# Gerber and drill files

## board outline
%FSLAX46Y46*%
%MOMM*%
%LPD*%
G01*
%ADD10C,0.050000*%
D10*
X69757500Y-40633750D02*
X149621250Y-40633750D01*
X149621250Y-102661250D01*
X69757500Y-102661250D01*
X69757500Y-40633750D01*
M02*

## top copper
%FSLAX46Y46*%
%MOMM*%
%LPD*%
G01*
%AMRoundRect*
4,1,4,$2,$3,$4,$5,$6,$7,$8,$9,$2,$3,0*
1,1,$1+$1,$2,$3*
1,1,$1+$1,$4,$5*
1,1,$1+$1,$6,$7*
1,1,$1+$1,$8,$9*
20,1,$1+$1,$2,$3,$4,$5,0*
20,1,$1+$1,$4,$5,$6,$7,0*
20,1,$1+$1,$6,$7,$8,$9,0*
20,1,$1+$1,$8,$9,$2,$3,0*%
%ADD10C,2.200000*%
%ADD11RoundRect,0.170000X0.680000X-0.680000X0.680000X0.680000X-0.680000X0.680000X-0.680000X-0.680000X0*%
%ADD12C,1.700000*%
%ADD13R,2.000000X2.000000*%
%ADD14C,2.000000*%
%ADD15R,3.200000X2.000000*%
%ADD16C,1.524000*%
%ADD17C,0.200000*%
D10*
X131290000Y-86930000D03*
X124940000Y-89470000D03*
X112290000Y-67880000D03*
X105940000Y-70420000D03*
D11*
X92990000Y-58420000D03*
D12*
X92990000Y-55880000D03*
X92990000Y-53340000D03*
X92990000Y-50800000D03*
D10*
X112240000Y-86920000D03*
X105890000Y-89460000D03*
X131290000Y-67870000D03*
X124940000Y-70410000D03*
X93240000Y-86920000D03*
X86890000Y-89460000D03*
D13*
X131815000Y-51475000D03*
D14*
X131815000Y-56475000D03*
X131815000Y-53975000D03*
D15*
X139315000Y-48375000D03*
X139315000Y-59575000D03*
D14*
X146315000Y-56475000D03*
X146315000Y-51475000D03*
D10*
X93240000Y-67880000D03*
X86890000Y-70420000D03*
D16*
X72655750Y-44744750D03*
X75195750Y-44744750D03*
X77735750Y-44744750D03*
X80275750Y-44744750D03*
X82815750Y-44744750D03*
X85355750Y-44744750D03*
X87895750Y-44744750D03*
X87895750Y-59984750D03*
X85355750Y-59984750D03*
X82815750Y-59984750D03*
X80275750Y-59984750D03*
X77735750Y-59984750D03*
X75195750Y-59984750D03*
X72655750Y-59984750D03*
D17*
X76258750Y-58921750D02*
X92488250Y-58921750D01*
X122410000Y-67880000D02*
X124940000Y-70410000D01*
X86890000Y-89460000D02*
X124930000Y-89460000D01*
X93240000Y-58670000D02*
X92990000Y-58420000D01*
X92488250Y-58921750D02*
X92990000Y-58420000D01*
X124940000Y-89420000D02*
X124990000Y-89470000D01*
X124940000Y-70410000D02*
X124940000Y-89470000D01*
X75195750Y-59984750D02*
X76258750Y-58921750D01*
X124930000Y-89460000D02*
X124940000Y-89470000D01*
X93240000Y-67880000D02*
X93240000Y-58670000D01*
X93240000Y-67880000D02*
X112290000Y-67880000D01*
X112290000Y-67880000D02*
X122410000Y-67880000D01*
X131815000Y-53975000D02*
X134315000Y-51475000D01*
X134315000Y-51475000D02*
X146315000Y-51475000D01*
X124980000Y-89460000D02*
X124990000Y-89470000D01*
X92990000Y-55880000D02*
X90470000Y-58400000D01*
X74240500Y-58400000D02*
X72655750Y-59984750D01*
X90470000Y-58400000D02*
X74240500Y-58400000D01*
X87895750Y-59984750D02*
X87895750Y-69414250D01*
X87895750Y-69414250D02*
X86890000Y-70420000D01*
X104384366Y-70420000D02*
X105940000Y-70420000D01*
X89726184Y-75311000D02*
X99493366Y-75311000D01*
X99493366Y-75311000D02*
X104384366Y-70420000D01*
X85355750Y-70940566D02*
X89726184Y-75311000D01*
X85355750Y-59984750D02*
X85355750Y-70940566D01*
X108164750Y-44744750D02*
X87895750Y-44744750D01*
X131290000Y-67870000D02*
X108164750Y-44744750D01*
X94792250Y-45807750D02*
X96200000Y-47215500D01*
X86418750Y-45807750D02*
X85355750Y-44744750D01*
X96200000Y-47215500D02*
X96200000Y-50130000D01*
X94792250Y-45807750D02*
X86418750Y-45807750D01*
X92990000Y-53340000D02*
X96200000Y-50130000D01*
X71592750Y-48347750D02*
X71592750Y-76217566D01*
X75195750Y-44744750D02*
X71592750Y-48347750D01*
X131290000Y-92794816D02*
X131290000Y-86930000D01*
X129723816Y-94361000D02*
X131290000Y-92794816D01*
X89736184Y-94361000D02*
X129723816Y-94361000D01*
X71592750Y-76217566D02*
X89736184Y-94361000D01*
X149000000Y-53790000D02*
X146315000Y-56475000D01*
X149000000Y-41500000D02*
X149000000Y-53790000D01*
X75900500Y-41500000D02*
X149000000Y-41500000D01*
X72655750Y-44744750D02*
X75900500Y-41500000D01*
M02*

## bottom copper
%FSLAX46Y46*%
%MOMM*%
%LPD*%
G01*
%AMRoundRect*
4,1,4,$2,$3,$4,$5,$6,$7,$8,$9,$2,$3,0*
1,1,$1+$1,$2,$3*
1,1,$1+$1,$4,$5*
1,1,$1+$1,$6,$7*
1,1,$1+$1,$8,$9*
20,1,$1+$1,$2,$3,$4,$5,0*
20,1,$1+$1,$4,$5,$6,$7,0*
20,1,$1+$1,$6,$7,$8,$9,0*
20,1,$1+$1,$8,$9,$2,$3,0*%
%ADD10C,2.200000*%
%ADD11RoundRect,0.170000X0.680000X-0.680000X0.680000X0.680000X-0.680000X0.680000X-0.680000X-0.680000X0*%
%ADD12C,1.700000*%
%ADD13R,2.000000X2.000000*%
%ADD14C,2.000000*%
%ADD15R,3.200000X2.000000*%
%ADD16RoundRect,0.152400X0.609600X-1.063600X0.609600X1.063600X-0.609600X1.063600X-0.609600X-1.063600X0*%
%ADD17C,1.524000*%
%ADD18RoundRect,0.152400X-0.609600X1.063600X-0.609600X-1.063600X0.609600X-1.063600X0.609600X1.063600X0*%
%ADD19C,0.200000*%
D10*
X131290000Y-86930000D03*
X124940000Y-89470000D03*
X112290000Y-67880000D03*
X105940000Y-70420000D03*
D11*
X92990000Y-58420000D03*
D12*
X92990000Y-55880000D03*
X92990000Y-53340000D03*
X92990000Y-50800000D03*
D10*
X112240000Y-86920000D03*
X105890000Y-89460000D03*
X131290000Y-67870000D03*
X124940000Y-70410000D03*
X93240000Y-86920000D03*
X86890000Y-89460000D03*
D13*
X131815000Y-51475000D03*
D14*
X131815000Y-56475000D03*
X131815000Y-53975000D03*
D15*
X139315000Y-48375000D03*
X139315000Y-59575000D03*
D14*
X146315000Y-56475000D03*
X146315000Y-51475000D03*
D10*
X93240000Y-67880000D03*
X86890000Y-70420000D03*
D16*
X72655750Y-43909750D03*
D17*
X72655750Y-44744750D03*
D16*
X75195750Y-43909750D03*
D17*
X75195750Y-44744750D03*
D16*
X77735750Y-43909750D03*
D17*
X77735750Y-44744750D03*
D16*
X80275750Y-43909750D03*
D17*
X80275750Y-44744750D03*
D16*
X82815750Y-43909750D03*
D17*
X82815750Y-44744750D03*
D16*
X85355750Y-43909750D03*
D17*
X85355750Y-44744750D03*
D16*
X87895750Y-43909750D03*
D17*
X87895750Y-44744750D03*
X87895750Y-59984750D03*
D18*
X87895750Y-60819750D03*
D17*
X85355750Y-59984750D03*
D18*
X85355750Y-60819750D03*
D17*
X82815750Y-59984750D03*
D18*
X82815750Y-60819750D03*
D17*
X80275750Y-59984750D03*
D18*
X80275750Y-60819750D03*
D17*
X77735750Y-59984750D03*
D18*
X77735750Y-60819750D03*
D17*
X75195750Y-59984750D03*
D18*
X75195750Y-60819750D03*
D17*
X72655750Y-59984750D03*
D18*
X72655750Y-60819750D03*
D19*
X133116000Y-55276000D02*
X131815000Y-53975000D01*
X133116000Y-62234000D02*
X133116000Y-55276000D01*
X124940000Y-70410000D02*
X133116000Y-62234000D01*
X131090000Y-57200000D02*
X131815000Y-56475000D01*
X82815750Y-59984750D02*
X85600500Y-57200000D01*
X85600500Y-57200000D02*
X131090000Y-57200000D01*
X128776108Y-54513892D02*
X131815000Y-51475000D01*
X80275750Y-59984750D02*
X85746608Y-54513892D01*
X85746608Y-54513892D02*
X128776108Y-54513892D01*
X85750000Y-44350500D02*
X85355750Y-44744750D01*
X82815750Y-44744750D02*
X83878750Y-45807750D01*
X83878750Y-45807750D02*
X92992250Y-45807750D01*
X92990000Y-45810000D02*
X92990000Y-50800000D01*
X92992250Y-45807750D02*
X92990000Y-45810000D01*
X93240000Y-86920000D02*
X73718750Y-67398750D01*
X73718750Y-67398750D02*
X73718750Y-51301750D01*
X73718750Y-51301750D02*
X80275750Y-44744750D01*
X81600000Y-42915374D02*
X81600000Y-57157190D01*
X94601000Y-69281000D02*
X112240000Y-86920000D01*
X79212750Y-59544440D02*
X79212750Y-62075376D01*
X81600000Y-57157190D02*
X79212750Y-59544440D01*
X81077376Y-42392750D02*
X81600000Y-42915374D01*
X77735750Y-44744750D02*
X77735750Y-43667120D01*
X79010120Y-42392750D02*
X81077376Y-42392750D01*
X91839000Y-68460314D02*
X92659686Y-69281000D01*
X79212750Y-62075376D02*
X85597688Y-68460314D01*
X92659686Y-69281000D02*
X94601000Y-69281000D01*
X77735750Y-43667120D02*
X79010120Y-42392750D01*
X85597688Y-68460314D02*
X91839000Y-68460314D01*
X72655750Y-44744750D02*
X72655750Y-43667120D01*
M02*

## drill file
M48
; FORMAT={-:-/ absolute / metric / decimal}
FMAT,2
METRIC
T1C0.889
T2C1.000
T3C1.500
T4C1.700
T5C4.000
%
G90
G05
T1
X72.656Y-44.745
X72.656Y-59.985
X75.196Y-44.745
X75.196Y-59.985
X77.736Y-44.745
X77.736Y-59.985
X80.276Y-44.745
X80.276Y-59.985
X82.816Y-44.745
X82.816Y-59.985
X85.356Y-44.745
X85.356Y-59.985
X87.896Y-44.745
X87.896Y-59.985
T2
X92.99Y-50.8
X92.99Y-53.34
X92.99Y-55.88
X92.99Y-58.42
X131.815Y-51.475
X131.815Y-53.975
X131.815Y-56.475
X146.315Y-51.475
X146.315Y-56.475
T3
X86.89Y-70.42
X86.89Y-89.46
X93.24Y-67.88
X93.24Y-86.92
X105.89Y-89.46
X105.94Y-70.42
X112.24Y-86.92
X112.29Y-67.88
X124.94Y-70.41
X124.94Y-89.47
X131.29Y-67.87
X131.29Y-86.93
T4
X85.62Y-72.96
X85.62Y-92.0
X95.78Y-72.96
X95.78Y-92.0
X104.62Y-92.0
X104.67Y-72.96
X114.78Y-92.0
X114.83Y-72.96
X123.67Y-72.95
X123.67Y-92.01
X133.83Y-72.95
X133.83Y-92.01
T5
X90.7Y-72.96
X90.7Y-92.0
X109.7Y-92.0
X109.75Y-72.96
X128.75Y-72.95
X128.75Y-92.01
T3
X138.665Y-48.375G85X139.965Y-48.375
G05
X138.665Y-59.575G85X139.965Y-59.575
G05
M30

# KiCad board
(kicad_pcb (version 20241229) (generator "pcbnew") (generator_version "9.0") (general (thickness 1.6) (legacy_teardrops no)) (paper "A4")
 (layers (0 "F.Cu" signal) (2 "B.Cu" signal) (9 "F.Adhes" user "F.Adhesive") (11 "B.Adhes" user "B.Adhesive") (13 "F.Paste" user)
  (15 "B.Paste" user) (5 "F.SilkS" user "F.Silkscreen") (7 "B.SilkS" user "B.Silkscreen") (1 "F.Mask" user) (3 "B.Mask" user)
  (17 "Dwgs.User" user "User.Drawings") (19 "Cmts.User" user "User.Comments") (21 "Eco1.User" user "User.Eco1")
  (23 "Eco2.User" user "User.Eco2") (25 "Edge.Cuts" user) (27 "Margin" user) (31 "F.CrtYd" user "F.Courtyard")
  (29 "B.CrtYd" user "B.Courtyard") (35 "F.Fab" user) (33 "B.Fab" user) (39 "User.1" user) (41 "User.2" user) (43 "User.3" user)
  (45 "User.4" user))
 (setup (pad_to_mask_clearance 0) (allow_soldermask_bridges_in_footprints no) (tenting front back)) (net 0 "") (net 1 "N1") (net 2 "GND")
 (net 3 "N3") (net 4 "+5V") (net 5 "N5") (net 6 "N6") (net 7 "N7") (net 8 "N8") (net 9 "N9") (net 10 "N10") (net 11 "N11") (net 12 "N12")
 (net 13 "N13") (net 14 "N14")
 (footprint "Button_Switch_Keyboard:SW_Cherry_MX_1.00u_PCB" (layer "F.Cu") (at 131.29 86.93)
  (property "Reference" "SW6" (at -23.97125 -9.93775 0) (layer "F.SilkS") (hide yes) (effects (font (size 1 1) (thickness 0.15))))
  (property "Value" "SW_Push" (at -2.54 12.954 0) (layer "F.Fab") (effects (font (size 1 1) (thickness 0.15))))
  (pad "" np_thru_hole circle (at -7.62 5.08) (size 1.7 1.7) (drill 1.7) (layers "*.Cu" "*.Mask"))
  (pad "" np_thru_hole circle (at -2.54 5.08) (size 4 4) (drill 4) (layers "*.Cu" "*.Mask"))
  (pad "" np_thru_hole circle (at 2.54 5.08) (size 1.7 1.7) (drill 1.7) (layers "*.Cu" "*.Mask"))
  (pad "1" thru_hole circle (at 0 0) (size 2.2 2.2) (drill 1.5) (layers "*.Cu" "*.Mask") (remove_unused_layers no) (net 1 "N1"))
  (pad "2" thru_hole circle (at -6.35 2.54) (size 2.2 2.2) (drill 1.5) (layers "*.Cu" "*.Mask") (remove_unused_layers no) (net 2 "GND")))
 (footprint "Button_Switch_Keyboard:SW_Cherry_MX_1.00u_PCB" (layer "F.Cu") (at 112.29 67.88)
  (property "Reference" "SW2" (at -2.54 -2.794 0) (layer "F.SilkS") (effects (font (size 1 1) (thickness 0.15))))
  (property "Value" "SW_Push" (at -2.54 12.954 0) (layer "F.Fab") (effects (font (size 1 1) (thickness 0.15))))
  (pad "" np_thru_hole circle (at -7.62 5.08) (size 1.7 1.7) (drill 1.7) (layers "*.Cu" "*.Mask"))
  (pad "" np_thru_hole circle (at -2.54 5.08) (size 4 4) (drill 4) (layers "*.Cu" "*.Mask"))
  (pad "" np_thru_hole circle (at 2.54 5.08) (size 1.7 1.7) (drill 1.7) (layers "*.Cu" "*.Mask"))
  (pad "1" thru_hole circle (at 0 0) (size 2.2 2.2) (drill 1.5) (layers "*.Cu" "*.Mask") (remove_unused_layers no) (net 2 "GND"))
  (pad "2" thru_hole circle (at -6.35 2.54) (size 2.2 2.2) (drill 1.5) (layers "*.Cu" "*.Mask") (remove_unused_layers no) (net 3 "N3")))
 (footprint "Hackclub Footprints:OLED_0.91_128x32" (layer "F.Cu") (at 92.99 58.42 90)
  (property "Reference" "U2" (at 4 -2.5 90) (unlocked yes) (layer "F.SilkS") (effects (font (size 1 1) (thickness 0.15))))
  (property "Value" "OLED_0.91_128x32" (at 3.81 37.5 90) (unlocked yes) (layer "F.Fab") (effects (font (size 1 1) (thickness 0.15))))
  (pad "1" thru_hole roundrect (at 0 0 90) (size 1.7 1.7) (drill 1) (layers "*.Cu" "*.Mask") (remove_unused_layers no)
   (roundrect_rratio 0.1) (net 2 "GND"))
  (pad "2" thru_hole circle (at 2.54 0 90) (size 1.7 1.7) (drill 1) (layers "*.Cu" "*.Mask") (remove_unused_layers no) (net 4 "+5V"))
  (pad "3" thru_hole circle (at 5.08 0 90) (size 1.7 1.7) (drill 1) (layers "*.Cu" "*.Mask") (remove_unused_layers no) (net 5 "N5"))
  (pad "4" thru_hole circle (at 7.62 0 90) (size 1.7 1.7) (drill 1) (layers "*.Cu" "*.Mask") (remove_unused_layers no) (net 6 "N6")))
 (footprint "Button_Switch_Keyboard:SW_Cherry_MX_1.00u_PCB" (layer "F.Cu") (at 112.24 86.92)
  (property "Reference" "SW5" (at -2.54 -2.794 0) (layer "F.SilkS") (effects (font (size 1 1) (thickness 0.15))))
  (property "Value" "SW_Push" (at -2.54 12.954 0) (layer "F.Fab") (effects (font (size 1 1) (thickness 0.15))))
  (pad "" np_thru_hole circle (at -7.62 5.08) (size 1.7 1.7) (drill 1.7) (layers "*.Cu" "*.Mask"))
  (pad "" np_thru_hole circle (at -2.54 5.08) (size 4 4) (drill 4) (layers "*.Cu" "*.Mask"))
  (pad "" np_thru_hole circle (at 2.54 5.08) (size 1.7 1.7) (drill 1.7) (layers "*.Cu" "*.Mask"))
  (pad "1" thru_hole circle (at 0 0) (size 2.2 2.2) (drill 1.5) (layers "*.Cu" "*.Mask") (remove_unused_layers no) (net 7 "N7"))
  (pad "2" thru_hole circle (at -6.35 2.54) (size 2.2 2.2) (drill 1.5) (layers "*.Cu" "*.Mask") (remove_unused_layers no) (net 2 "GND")))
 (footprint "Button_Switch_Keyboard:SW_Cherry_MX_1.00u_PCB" (layer "F.Cu") (at 131.29 67.87)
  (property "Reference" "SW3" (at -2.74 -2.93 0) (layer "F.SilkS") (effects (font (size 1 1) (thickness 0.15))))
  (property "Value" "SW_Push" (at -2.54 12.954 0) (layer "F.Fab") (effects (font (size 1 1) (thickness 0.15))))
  (pad "" np_thru_hole circle (at -7.62 5.08) (size 1.7 1.7) (drill 1.7) (layers "*.Cu" "*.Mask"))
  (pad "" np_thru_hole circle (at -2.54 5.08) (size 4 4) (drill 4) (layers "*.Cu" "*.Mask"))
  (pad "" np_thru_hole circle (at 2.54 5.08) (size 1.7 1.7) (drill 1.7) (layers "*.Cu" "*.Mask"))
  (pad "1" thru_hole circle (at 0 0) (size 2.2 2.2) (drill 1.5) (layers "*.Cu" "*.Mask") (remove_unused_layers no) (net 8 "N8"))
  (pad "2" thru_hole circle (at -6.35 2.54) (size 2.2 2.2) (drill 1.5) (layers "*.Cu" "*.Mask") (remove_unused_layers no) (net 2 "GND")))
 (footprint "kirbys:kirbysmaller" (layer "F.Cu") (at 80 51.5)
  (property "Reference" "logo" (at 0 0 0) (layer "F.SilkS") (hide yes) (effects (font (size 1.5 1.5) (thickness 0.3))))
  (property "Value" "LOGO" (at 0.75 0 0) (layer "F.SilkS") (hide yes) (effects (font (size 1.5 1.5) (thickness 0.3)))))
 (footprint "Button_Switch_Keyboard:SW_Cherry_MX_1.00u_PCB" (layer "F.Cu") (at 93.24 86.92)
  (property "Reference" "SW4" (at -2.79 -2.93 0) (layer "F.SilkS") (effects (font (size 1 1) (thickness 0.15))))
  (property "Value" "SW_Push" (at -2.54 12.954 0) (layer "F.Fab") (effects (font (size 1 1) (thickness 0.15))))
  (pad "" np_thru_hole circle (at -7.62 5.08) (size 1.7 1.7) (drill 1.7) (layers "*.Cu" "*.Mask"))
  (pad "" np_thru_hole circle (at -2.54 5.08) (size 4 4) (drill 4) (layers "*.Cu" "*.Mask"))
  (pad "" np_thru_hole circle (at 2.54 5.08) (size 1.7 1.7) (drill 1.7) (layers "*.Cu" "*.Mask"))
  (pad "1" thru_hole circle (at 0 0) (size 2.2 2.2) (drill 1.5) (layers "*.Cu" "*.Mask") (remove_unused_layers no) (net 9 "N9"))
  (pad "2" thru_hole circle (at -6.35 2.54) (size 2.2 2.2) (drill 1.5) (layers "*.Cu" "*.Mask") (remove_unused_layers no) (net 2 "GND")))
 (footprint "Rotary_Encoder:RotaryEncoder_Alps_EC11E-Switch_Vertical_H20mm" (layer "F.Cu") (at 131.815 51.475)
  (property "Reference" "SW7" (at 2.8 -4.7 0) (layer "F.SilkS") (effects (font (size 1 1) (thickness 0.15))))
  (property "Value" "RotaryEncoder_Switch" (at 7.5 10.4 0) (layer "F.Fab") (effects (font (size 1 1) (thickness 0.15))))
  (pad "A" thru_hole rect (at 0 0) (size 2 2) (drill 1) (layers "*.Cu" "*.Mask") (remove_unused_layers no) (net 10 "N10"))
  (pad "B" thru_hole circle (at 0 5) (size 2 2) (drill 1) (layers "*.Cu" "*.Mask") (remove_unused_layers no) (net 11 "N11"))
  (pad "C" thru_hole circle (at 0 2.5) (size 2 2) (drill 1) (layers "*.Cu" "*.Mask") (remove_unused_layers no) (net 2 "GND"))
  (pad "MP" thru_hole rect (at 7.5 -3.1) (size 3.2 2) (drill oval 2.8 1.5) (layers "*.Cu" "*.Mask") (remove_unused_layers no))
  (pad "MP" thru_hole rect (at 7.5 8.1) (size 3.2 2) (drill oval 2.8 1.5) (layers "*.Cu" "*.Mask") (remove_unused_layers no))
  (pad "S1" thru_hole circle (at 14.5 5) (size 2 2) (drill 1) (layers "*.Cu" "*.Mask") (remove_unused_layers no) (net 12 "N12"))
  (pad "S2" thru_hole circle (at 14.5 0) (size 2 2) (drill 1) (layers "*.Cu" "*.Mask") (remove_unused_layers no) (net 2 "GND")))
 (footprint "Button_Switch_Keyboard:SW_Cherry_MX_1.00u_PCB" (layer "F.Cu") (at 93.24 67.88)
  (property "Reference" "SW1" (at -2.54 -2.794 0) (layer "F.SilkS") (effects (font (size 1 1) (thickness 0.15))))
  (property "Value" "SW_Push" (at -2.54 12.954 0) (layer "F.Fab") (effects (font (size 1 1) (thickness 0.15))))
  (pad "" np_thru_hole circle (at -7.62 5.08) (size 1.7 1.7) (drill 1.7) (layers "*.Cu" "*.Mask"))
  (pad "" np_thru_hole circle (at -2.54 5.08) (size 4 4) (drill 4) (layers "*.Cu" "*.Mask"))
  (pad "" np_thru_hole circle (at 2.54 5.08) (size 1.7 1.7) (drill 1.7) (layers "*.Cu" "*.Mask"))
  (pad "1" thru_hole circle (at 0 0) (size 2.2 2.2) (drill 1.5) (layers "*.Cu" "*.Mask") (remove_unused_layers no) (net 2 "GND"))
  (pad "2" thru_hole circle (at -6.35 2.54) (size 2.2 2.2) (drill 1.5) (layers "*.Cu" "*.Mask") (remove_unused_layers no) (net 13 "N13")))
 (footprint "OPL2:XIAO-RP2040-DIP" (layer "B.Cu") (at 80.27575 52.36475 -90)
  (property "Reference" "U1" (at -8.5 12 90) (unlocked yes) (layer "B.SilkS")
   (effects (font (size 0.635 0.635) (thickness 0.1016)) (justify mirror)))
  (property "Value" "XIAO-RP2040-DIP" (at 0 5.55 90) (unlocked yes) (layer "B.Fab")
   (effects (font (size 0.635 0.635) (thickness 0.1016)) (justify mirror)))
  (pad "1" smd roundrect (at -8.455 7.62 90) (size 2.432 1.524) (layers "B.Cu" "B.Mask") (roundrect_rratio 0.1) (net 12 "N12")
   (thermal_bridge_angle 45))
  (pad "1" thru_hole circle (at -7.62 7.62 90) (size 1.524 1.524) (drill 0.889) (layers "*.Cu" "*.Mask") (remove_unused_layers no)
   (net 12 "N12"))
  (pad "2" smd roundrect (at -8.455 5.08 90) (size 2.432 1.524) (layers "B.Cu" "B.Mask") (roundrect_rratio 0.1) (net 1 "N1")
   (thermal_bridge_angle 45))
  (pad "2" thru_hole circle (at -7.62 5.08 90) (size 1.524 1.524) (drill 0.889) (layers "*.Cu" "*.Mask") (remove_unused_layers no)
   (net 1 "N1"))
  (pad "3" smd roundrect (at -8.455 2.54 90) (size 2.432 1.524) (layers "B.Cu" "B.Mask") (roundrect_rratio 0.1) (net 7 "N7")
   (thermal_bridge_angle 45))
  (pad "3" thru_hole circle (at -7.62 2.54 90) (size 1.524 1.524) (drill 0.889) (layers "*.Cu" "*.Mask") (remove_unused_layers no)
   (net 7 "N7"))
  (pad "4" smd roundrect (at -8.455 0 90) (size 2.432 1.524) (layers "B.Cu" "B.Mask") (roundrect_rratio 0.1) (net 9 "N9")
   (thermal_bridge_angle 45))
  (pad "4" thru_hole circle (at -7.62 0 90) (size 1.524 1.524) (drill 0.889) (layers "*.Cu" "*.Mask") (remove_unused_layers no) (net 9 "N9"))
  (pad "5" smd roundrect (at -8.455 -2.54 90) (size 2.432 1.524) (layers "B.Cu" "B.Mask") (roundrect_rratio 0.1) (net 6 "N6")
   (thermal_bridge_angle 45))
  (pad "5" thru_hole circle (at -7.62 -2.54 90) (size 1.524 1.524) (drill 0.889) (layers "*.Cu" "*.Mask") (remove_unused_layers no)
   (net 6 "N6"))
  (pad "6" smd roundrect (at -8.455 -5.08 90) (size 2.432 1.524) (layers "B.Cu" "B.Mask") (roundrect_rratio 0.1) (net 5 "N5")
   (thermal_bridge_angle 45))
  (pad "6" thru_hole circle (at -7.62 -5.08 90) (size 1.524 1.524) (drill 0.889) (layers "*.Cu" "*.Mask") (remove_unused_layers no)
   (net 5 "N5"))
  (pad "7" smd roundrect (at -8.455 -7.62 90) (size 2.432 1.524) (layers "B.Cu" "B.Mask") (roundrect_rratio 0.1) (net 8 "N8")
   (thermal_bridge_angle 45))
  (pad "7" thru_hole circle (at -7.62 -7.62 90) (size 1.524 1.524) (drill 0.889) (layers "*.Cu" "*.Mask") (remove_unused_layers no)
   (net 8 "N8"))
  (pad "8" thru_hole circle (at 7.62 -7.62 270) (size 1.524 1.524) (drill 0.889) (layers "*.Cu" "*.Mask") (remove_unused_layers no)
   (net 13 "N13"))
  (pad "8" smd roundrect (at 8.455 -7.62 270) (size 2.432 1.524) (layers "B.Cu" "B.Mask") (roundrect_rratio 0.1) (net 13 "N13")
   (thermal_bridge_angle 45))
  (pad "9" thru_hole circle (at 7.62 -5.08 270) (size 1.524 1.524) (drill 0.889) (layers "*.Cu" "*.Mask") (remove_unused_layers no)
   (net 3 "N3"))
  (pad "9" smd roundrect (at 8.455 -5.08 270) (size 2.432 1.524) (layers "B.Cu" "B.Mask") (roundrect_rratio 0.1) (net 3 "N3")
   (thermal_bridge_angle 45))
  (pad "10" thru_hole circle (at 7.62 -2.54 270) (size 1.524 1.524) (drill 0.889) (layers "*.Cu" "*.Mask") (remove_unused_layers no)
   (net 11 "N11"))
  (pad "10" smd roundrect (at 8.455 -2.54 270) (size 2.432 1.524) (layers "B.Cu" "B.Mask") (roundrect_rratio 0.1) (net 11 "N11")
   (thermal_bridge_angle 45))
  (pad "11" thru_hole circle (at 7.62 0 270) (size 1.524 1.524) (drill 0.889) (layers "*.Cu" "*.Mask") (remove_unused_layers no)
   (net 10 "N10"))
  (pad "11" smd roundrect (at 8.455 0 270) (size 2.432 1.524) (layers "B.Cu" "B.Mask") (roundrect_rratio 0.1) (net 10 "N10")
   (thermal_bridge_angle 45))
  (pad "12" thru_hole circle (at 7.62 2.54 270) (size 1.524 1.524) (drill 0.889) (layers "*.Cu" "*.Mask") (remove_unused_layers no)
   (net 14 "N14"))
  (pad "12" smd roundrect (at 8.455 2.54 270) (size 2.432 1.524) (layers "B.Cu" "B.Mask") (roundrect_rratio 0.1) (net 14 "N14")
   (thermal_bridge_angle 45))
  (pad "13" thru_hole circle (at 7.62 5.08 270) (size 1.524 1.524) (drill 0.889) (layers "*.Cu" "*.Mask") (remove_unused_layers no)
   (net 2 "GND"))
  (pad "13" smd roundrect (at 8.455 5.08 270) (size 2.432 1.524) (layers "B.Cu" "B.Mask") (roundrect_rratio 0.1) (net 2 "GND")
   (thermal_bridge_angle 45))
  (pad "14" thru_hole circle (at 7.62 7.62 270) (size 1.524 1.524) (drill 0.889) (layers "*.Cu" "*.Mask") (remove_unused_layers no)
   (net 4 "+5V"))
  (pad "14" smd roundrect (at 8.455 7.62 270) (size 2.432 1.524) (layers "B.Cu" "B.Mask") (roundrect_rratio 0.1) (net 4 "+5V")
   (thermal_bridge_angle 45)))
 (gr_rect (start 69.7575 40.63375) (end 149.62125 102.66125) (stroke (width 0.05) (type default)) (fill no) (layer "Edge.Cuts"))
 (segment (start 76.25875 58.92175) (end 92.48825 58.92175) (width 0.2) (layer "F.Cu") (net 2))
 (segment (start 122.41 67.88) (end 124.94 70.41) (width 0.2) (layer "F.Cu") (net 2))
 (segment (start 86.89 89.46) (end 124.93 89.46) (width 0.2) (layer "F.Cu") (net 2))
 (segment (start 93.24 58.67) (end 92.99 58.42) (width 0.2) (layer "F.Cu") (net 2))
 (segment (start 92.48825 58.92175) (end 92.99 58.42) (width 0.2) (layer "F.Cu") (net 2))
 (segment (start 124.94 89.42) (end 124.99 89.47) (width 0.2) (layer "F.Cu") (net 2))
 (segment (start 124.94 70.41) (end 124.94 89.47) (width 0.2) (layer "F.Cu") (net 2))
 (segment (start 75.19575 59.98475) (end 76.25875 58.92175) (width 0.2) (layer "F.Cu") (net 2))
 (segment (start 124.93 89.46) (end 124.94 89.47) (width 0.2) (layer "F.Cu") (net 2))
 (segment (start 93.24 67.88) (end 93.24 58.67) (width 0.2) (layer "F.Cu") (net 2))
 (segment (start 93.24 67.88) (end 112.29 67.88) (width 0.2) (layer "F.Cu") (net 2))
 (segment (start 112.29 67.88) (end 122.41 67.88) (width 0.2) (layer "F.Cu") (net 2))
 (segment (start 131.815 53.975) (end 134.315 51.475) (width 0.2) (layer "F.Cu") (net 2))
 (segment (start 134.315 51.475) (end 146.315 51.475) (width 0.2) (layer "F.Cu") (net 2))
 (segment (start 124.98 89.46) (end 124.99 89.47) (width 0.2) (layer "F.Cu") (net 2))
 (segment (start 133.116 55.276) (end 131.815 53.975) (width 0.2) (layer "B.Cu") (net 2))
 (segment (start 133.116 62.234) (end 133.116 55.276) (width 0.2) (layer "B.Cu") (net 2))
 (segment (start 124.94 70.41) (end 133.116 62.234) (width 0.2) (layer "B.Cu") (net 2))
 (segment (start 92.99 55.88) (end 90.47 58.4) (width 0.2) (layer "F.Cu") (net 4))
 (segment (start 74.2405 58.4) (end 72.65575 59.98475) (width 0.2) (layer "F.Cu") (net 4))
 (segment (start 90.47 58.4) (end 74.2405 58.4) (width 0.2) (layer "F.Cu") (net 4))
 (segment (start 87.89575 59.98475) (end 87.89575 69.41425) (width 0.2) (layer "F.Cu") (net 13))
 (segment (start 87.89575 69.41425) (end 86.89 70.42) (width 0.2) (layer "F.Cu") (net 13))
 (segment (start 104.384366 70.42) (end 105.94 70.42) (width 0.2) (layer "F.Cu") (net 3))
 (segment (start 89.726184 75.311) (end 99.493366 75.311) (width 0.2) (layer "F.Cu") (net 3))
 (segment (start 99.493366 75.311) (end 104.384366 70.42) (width 0.2) (layer "F.Cu") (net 3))
 (segment (start 85.35575 70.940566) (end 89.726184 75.311) (width 0.2) (layer "F.Cu") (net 3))
 (segment (start 85.35575 59.98475) (end 85.35575 70.940566) (width 0.2) (layer "F.Cu") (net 3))
 (segment (start 131.09 57.2) (end 131.815 56.475) (width 0.2) (layer "B.Cu") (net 11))
 (segment (start 82.81575 59.98475) (end 85.6005 57.2) (width 0.2) (layer "B.Cu") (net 11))
 (segment (start 85.6005 57.2) (end 131.09 57.2) (width 0.2) (layer "B.Cu") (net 11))
 (segment (start 128.776108 54.513892) (end 131.815 51.475) (width 0.2) (layer "B.Cu") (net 10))
 (segment (start 80.27575 59.98475) (end 85.746608 54.513892) (width 0.2) (layer "B.Cu") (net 10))
 (segment (start 85.746608 54.513892) (end 128.776108 54.513892) (width 0.2) (layer "B.Cu") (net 10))
 (segment (start 108.16475 44.74475) (end 87.89575 44.74475) (width 0.2) (layer "F.Cu") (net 8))
 (segment (start 131.29 67.87) (end 108.16475 44.74475) (width 0.2) (layer "F.Cu") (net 8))
 (segment (start 94.79225 45.80775) (end 96.2 47.2155) (width 0.2) (layer "F.Cu") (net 5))
 (segment (start 86.41875 45.80775) (end 85.35575 44.74475) (width 0.2) (layer "F.Cu") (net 5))
 (segment (start 96.2 47.2155) (end 96.2 50.13) (width 0.2) (layer "F.Cu") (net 5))
 (segment (start 94.79225 45.80775) (end 86.41875 45.80775) (width 0.2) (layer "F.Cu") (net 5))
 (segment (start 92.99 53.34) (end 96.2 50.13) (width 0.2) (layer "F.Cu") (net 5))
 (segment (start 85.75 44.3505) (end 85.35575 44.74475) (width 0.2) (layer "B.Cu") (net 5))
 (segment (start 82.81575 44.74475) (end 83.87875 45.80775) (width 0.2) (layer "B.Cu") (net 6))
 (segment (start 83.87875 45.80775) (end 92.99225 45.80775) (width 0.2) (layer "B.Cu") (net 6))
 (segment (start 92.99 45.81) (end 92.99 50.8) (width 0.2) (layer "B.Cu") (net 6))
 (segment (start 92.99225 45.80775) (end 92.99 45.81) (width 0.2) (layer "B.Cu") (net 6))
 (segment (start 93.24 86.92) (end 73.71875 67.39875) (width 0.2) (layer "B.Cu") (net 9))
 (segment (start 73.71875 67.39875) (end 73.71875 51.30175) (width 0.2) (layer "B.Cu") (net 9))
 (segment (start 73.71875 51.30175) (end 80.27575 44.74475) (width 0.2) (layer "B.Cu") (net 9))
 (segment (start 81.6 42.915374) (end 81.6 57.15719) (width 0.2) (layer "B.Cu") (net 7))
 (segment (start 94.601 69.281) (end 112.24 86.92) (width 0.2) (layer "B.Cu") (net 7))
 (segment (start 79.21275 59.54444) (end 79.21275 62.075376) (width 0.2) (layer "B.Cu") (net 7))
 (segment (start 81.6 57.15719) (end 79.21275 59.54444) (width 0.2) (layer "B.Cu") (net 7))
 (segment (start 81.077376 42.39275) (end 81.6 42.915374) (width 0.2) (layer "B.Cu") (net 7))
 (segment (start 77.73575 44.74475) (end 77.73575 43.66712) (width 0.2) (layer "B.Cu") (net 7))
 (segment (start 79.01012 42.39275) (end 81.077376 42.39275) (width 0.2) (layer "B.Cu") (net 7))
 (segment (start 91.839 68.460314) (end 92.659686 69.281) (width 0.2) (layer "B.Cu") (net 7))
 (segment (start 79.21275 62.075376) (end 85.597688 68.460314) (width 0.2) (layer "B.Cu") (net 7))
 (segment (start 92.659686 69.281) (end 94.601 69.281) (width 0.2) (layer "B.Cu") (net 7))
 (segment (start 77.73575 43.66712) (end 79.01012 42.39275) (width 0.2) (layer "B.Cu") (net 7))
 (segment (start 85.597688 68.460314) (end 91.839 68.460314) (width 0.2) (layer "B.Cu") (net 7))
 (segment (start 71.59275 48.34775) (end 71.59275 76.217566) (width 0.2) (layer "F.Cu") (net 1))
 (segment (start 75.19575 44.74475) (end 71.59275 48.34775) (width 0.2) (layer "F.Cu") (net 1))
 (segment (start 131.29 92.794816) (end 131.29 86.93) (width 0.2) (layer "F.Cu") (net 1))
 (segment (start 129.723816 94.361) (end 131.29 92.794816) (width 0.2) (layer "F.Cu") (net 1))
 (segment (start 89.736184 94.361) (end 129.723816 94.361) (width 0.2) (layer "F.Cu") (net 1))
 (segment (start 71.59275 76.217566) (end 89.736184 94.361) (width 0.2) (layer "F.Cu") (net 1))
 (segment (start 149 53.79) (end 146.315 56.475) (width 0.2) (layer "F.Cu") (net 12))
 (segment (start 149 41.5) (end 149 53.79) (width 0.2) (layer "F.Cu") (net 12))
 (segment (start 75.9005 41.5) (end 149 41.5) (width 0.2) (layer "F.Cu") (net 12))
 (segment (start 72.65575 44.74475) (end 75.9005 41.5) (width 0.2) (layer "F.Cu") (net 12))
 (segment (start 72.65575 44.74475) (end 72.65575 43.66712) (width 0.2) (layer "B.Cu") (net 12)))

